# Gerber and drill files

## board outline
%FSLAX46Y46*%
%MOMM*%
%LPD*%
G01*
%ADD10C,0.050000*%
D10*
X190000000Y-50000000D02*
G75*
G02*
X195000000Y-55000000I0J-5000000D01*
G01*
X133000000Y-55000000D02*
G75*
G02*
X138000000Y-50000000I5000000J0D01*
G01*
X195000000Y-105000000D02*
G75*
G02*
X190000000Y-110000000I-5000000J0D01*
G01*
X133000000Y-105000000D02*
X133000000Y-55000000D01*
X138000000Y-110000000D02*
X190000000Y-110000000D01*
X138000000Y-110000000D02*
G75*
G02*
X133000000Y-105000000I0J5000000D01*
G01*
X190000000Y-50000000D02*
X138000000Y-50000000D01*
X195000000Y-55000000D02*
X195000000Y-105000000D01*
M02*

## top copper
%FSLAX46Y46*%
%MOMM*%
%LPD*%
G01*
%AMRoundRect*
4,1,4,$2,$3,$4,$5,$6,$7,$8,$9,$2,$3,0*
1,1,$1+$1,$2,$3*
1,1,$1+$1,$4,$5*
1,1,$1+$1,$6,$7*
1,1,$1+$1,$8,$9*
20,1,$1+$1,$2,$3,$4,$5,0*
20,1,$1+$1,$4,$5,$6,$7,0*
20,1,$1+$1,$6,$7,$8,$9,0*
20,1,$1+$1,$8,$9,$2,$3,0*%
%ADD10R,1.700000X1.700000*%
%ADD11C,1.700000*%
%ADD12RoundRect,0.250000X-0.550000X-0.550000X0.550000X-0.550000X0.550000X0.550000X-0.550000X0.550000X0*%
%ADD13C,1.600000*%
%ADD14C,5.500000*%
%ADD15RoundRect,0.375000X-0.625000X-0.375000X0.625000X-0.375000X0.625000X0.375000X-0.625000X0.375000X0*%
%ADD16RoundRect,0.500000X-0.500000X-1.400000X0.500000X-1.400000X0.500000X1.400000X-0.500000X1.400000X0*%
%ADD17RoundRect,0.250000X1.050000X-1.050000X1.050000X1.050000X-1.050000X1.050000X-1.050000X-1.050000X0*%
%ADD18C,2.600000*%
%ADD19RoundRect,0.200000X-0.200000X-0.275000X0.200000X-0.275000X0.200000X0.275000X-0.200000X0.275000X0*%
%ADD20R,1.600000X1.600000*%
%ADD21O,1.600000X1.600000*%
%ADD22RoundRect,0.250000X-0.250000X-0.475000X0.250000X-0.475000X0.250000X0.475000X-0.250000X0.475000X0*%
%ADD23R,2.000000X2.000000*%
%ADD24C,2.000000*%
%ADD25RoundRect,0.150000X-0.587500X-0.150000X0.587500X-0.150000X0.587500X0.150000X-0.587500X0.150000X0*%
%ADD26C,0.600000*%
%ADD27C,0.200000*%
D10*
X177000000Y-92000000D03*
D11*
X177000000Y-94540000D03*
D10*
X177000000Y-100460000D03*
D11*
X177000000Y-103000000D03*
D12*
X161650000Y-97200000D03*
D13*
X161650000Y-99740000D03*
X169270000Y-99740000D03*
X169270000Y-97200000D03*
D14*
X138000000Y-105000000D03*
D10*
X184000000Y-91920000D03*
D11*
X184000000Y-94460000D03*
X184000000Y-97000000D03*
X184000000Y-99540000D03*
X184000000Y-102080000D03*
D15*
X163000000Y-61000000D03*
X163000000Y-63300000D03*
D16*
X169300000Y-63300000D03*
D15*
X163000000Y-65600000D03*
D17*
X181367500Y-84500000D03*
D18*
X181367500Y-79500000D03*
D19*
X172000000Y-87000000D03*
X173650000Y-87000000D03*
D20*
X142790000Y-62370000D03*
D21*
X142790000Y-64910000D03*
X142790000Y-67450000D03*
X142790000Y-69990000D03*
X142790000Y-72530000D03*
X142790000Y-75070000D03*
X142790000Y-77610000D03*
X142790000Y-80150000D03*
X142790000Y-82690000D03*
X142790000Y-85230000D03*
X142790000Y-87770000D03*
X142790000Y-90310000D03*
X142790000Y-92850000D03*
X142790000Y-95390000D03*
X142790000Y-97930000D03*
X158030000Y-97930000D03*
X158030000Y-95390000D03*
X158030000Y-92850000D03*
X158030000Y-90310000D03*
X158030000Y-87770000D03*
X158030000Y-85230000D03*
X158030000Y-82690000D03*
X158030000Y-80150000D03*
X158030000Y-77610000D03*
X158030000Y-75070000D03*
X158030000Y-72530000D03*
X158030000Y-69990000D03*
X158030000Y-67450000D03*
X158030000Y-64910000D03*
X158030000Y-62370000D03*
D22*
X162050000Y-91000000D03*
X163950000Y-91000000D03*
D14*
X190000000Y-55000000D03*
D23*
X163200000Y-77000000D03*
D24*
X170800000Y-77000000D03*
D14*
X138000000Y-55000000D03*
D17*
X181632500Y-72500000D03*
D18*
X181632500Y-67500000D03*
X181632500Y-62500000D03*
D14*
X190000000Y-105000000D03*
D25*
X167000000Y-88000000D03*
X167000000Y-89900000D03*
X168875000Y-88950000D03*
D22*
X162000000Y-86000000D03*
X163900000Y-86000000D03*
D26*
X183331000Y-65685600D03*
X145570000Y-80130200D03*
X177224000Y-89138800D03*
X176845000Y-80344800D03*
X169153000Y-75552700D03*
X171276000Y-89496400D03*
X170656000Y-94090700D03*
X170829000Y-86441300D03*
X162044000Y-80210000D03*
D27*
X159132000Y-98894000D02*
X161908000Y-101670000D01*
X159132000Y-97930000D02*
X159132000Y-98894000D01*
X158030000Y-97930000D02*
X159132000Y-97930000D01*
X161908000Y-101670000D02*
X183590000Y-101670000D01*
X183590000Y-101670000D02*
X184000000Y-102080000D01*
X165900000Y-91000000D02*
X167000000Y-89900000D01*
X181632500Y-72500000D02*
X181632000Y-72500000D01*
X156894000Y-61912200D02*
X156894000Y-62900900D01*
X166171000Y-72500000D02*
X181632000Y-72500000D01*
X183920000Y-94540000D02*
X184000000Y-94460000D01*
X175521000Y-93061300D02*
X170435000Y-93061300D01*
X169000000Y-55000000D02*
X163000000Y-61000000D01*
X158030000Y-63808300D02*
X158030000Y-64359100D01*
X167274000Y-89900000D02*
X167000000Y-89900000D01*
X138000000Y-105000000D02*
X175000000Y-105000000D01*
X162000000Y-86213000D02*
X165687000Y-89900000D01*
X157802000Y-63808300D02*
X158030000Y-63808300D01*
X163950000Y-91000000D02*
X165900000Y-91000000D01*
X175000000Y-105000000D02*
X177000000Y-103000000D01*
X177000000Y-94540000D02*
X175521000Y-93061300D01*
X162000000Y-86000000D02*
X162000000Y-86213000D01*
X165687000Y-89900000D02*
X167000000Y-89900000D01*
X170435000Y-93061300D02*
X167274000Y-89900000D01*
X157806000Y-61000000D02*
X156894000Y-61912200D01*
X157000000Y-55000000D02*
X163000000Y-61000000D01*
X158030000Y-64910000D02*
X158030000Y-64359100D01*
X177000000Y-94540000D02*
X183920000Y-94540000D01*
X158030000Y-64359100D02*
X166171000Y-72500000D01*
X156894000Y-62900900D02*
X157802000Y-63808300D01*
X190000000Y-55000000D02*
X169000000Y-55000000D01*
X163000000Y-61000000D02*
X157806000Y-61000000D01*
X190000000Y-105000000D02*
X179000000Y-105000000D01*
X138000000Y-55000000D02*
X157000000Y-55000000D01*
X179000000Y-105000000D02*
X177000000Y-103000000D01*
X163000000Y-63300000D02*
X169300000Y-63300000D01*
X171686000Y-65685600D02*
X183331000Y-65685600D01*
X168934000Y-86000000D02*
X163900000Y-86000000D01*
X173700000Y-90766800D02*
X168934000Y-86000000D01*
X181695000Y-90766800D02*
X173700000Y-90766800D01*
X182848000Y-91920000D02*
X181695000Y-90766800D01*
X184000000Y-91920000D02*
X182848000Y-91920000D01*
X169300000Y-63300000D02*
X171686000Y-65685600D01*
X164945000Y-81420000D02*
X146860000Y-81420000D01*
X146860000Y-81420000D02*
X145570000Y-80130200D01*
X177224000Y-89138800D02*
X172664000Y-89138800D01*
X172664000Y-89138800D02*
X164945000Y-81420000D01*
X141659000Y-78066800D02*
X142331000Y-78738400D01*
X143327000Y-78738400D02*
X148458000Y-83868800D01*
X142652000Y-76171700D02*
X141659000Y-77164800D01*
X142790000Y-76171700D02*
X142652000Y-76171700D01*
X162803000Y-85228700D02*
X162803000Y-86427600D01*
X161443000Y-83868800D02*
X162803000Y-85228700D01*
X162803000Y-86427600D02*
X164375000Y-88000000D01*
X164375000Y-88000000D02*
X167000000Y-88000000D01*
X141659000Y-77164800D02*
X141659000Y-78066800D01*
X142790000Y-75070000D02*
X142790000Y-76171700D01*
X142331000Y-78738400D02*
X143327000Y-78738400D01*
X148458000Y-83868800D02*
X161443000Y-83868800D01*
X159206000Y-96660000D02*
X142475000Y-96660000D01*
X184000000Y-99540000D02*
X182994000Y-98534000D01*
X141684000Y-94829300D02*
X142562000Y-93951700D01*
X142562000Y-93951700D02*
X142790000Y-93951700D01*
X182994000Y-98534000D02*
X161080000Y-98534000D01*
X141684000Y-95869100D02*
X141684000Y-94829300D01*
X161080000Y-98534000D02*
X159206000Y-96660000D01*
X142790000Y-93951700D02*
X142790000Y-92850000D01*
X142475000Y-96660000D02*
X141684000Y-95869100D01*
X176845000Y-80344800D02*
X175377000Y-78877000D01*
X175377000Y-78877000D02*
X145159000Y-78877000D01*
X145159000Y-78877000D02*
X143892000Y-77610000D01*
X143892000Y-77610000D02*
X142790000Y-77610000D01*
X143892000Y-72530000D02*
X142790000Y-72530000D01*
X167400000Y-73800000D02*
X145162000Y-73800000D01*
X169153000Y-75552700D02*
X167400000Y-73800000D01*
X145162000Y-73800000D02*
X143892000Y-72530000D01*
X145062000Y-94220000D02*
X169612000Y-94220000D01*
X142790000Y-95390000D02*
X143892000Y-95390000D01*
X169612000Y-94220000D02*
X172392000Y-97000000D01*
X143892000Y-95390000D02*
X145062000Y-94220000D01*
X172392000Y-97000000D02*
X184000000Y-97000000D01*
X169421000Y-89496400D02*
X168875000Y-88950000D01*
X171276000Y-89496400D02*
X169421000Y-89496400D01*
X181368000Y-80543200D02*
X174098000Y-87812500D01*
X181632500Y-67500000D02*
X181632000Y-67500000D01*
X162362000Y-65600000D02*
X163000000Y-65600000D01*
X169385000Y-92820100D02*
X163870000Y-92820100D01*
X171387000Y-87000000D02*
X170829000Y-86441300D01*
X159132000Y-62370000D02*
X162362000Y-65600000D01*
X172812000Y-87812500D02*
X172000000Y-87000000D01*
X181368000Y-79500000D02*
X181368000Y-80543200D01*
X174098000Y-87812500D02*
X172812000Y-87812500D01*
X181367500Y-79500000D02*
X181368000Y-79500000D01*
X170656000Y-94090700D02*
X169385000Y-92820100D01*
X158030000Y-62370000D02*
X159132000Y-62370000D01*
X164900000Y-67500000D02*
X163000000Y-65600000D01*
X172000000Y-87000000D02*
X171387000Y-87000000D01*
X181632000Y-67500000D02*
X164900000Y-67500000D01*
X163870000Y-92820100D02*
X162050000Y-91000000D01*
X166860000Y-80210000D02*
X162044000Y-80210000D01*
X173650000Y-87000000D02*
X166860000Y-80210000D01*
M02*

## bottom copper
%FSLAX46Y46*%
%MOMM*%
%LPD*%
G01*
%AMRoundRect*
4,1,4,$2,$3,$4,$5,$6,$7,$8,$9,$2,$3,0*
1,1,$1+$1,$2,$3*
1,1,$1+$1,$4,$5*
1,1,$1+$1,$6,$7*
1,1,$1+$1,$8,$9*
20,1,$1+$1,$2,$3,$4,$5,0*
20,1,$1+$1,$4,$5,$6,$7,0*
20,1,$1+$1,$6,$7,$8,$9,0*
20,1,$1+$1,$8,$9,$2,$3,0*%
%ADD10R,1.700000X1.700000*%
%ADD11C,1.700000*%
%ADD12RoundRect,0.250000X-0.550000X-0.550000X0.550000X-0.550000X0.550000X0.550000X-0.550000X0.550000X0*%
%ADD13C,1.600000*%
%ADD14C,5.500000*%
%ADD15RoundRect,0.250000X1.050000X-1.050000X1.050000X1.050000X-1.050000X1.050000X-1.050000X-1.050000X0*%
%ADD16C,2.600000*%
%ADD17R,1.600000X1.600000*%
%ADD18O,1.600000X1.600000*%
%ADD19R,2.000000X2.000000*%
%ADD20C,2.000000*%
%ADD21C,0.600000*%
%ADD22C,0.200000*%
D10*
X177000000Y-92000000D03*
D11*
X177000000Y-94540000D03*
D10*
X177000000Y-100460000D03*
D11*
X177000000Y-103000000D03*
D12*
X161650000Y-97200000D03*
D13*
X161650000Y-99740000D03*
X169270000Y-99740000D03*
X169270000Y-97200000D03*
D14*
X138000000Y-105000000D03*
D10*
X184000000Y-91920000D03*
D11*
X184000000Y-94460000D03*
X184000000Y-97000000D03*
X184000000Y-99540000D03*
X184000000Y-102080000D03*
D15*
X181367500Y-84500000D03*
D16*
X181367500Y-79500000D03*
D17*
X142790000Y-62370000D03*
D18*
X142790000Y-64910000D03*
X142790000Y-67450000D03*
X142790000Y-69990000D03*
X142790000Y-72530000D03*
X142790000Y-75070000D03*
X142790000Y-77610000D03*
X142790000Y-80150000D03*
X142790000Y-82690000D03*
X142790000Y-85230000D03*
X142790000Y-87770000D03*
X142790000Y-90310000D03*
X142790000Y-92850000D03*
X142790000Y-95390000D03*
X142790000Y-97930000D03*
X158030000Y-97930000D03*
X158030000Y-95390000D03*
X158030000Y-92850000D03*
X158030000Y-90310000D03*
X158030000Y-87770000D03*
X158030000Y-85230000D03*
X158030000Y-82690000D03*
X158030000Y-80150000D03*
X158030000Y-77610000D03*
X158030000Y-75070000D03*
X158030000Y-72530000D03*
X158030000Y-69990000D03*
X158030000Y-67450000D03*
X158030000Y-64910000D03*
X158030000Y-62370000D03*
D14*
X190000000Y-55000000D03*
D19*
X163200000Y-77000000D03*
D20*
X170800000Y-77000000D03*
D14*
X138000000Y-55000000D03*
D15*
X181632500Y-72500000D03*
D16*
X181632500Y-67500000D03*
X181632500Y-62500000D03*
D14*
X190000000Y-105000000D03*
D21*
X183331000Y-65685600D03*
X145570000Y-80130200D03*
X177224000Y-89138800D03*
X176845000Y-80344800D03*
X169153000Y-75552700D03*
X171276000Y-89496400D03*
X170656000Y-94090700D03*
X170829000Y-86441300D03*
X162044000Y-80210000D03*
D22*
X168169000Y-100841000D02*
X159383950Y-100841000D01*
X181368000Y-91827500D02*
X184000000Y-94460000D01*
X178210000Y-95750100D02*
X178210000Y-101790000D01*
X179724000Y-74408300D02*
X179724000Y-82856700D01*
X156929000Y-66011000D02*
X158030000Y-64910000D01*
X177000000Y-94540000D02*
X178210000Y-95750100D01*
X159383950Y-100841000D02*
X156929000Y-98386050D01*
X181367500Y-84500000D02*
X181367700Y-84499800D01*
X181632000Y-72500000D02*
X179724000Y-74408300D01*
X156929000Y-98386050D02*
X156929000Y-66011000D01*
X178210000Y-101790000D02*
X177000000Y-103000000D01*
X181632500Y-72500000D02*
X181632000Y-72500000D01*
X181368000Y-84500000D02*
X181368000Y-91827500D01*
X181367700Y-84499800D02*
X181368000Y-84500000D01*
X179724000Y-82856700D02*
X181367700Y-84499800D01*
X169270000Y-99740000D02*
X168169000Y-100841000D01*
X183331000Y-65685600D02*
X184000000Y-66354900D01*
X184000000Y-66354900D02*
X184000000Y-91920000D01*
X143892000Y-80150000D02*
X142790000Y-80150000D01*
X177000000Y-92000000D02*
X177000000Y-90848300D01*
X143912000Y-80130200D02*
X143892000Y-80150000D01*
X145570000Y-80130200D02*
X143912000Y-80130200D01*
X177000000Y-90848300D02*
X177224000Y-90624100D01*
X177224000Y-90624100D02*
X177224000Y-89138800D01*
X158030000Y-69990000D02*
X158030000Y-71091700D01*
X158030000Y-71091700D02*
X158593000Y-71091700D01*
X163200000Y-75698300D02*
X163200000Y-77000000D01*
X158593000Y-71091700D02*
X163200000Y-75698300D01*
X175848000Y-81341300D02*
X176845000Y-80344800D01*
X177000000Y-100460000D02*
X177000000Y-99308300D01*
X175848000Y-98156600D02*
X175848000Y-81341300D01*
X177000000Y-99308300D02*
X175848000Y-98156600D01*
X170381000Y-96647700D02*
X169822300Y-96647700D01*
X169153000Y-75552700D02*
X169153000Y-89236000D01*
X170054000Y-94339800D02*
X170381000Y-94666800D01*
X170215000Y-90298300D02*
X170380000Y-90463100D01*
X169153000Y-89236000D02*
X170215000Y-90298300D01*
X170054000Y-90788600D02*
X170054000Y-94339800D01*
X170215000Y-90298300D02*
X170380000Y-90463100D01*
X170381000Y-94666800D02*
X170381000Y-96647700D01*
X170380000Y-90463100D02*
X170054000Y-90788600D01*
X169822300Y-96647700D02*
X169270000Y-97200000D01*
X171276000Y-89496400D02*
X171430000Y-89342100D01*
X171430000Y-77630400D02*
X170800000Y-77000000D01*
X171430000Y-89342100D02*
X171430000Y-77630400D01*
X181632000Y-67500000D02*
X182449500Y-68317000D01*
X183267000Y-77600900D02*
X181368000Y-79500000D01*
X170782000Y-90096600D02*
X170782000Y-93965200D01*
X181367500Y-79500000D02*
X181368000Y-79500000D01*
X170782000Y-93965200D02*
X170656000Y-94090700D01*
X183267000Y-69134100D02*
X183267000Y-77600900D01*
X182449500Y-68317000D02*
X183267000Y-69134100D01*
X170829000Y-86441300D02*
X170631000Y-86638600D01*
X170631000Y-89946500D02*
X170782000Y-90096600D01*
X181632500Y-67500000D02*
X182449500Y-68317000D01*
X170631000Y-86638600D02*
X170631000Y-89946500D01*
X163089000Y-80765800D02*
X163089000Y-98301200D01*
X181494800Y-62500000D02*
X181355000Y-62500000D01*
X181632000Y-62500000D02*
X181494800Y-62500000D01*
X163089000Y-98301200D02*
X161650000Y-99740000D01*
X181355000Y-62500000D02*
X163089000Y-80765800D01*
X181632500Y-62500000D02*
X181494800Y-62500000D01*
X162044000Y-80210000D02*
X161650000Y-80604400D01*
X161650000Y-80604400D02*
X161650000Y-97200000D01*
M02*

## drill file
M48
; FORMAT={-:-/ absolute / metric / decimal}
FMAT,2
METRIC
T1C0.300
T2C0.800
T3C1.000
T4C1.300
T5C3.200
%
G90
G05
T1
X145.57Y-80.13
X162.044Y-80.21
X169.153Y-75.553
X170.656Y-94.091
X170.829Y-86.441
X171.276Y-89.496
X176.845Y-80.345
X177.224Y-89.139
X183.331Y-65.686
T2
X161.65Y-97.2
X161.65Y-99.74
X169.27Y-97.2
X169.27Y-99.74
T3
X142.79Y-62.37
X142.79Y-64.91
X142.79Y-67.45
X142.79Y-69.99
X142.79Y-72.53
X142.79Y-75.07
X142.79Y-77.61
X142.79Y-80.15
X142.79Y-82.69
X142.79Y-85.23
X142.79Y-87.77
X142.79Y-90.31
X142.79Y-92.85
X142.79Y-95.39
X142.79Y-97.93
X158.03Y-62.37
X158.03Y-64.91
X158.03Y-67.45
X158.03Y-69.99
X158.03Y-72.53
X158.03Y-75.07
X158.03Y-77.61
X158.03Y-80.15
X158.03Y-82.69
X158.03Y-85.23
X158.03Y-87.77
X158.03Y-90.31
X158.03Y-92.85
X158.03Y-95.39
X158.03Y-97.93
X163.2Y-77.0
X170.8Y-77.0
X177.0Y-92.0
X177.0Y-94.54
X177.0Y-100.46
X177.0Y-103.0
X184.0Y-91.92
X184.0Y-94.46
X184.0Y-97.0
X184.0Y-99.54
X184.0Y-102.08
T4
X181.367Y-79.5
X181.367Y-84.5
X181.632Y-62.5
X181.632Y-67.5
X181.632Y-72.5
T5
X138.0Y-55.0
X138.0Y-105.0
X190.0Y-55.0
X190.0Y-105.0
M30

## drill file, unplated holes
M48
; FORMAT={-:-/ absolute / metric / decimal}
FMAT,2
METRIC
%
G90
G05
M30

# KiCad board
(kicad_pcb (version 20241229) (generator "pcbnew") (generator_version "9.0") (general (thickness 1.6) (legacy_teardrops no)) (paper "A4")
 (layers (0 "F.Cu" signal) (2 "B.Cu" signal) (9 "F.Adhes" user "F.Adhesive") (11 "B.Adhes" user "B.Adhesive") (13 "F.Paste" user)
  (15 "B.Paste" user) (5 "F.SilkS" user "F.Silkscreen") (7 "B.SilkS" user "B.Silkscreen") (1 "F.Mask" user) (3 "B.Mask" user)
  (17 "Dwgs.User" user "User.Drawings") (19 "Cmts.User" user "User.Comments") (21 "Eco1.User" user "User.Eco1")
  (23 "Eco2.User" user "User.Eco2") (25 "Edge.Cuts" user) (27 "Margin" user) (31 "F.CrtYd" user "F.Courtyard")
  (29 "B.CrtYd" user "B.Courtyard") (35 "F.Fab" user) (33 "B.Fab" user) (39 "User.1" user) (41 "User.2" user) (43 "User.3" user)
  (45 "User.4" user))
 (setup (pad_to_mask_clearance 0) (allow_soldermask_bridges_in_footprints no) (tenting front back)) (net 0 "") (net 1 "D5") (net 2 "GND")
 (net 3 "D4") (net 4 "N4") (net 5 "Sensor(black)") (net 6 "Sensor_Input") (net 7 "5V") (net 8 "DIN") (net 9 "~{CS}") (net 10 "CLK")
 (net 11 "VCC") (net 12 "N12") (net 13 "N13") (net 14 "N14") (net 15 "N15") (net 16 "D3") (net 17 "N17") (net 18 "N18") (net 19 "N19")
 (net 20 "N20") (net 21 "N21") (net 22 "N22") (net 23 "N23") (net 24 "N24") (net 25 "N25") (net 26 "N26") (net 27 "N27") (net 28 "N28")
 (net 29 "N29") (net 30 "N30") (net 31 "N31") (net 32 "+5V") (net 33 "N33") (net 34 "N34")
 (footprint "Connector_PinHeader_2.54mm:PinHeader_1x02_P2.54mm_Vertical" (layer "F.Cu") (at 177 92)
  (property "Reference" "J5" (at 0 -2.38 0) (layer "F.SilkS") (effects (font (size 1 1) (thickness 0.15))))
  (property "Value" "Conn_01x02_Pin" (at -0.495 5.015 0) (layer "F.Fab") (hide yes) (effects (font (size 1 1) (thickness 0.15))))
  (pad "1" thru_hole rect (at 0 0) (size 1.7 1.7) (drill 1) (layers "*.Cu" "*.Mask") (remove_unused_layers no) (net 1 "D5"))
  (pad "2" thru_hole circle (at 0 2.54) (size 1.7 1.7) (drill 1) (layers "*.Cu" "*.Mask") (remove_unused_layers no) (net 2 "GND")))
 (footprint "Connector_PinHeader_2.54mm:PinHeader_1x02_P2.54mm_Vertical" (layer "F.Cu") (at 177 100.46)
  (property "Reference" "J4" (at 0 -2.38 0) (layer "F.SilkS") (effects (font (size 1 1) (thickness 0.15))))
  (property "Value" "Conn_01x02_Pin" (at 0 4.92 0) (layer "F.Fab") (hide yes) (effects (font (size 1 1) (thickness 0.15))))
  (pad "1" thru_hole rect (at 0 0) (size 1.7 1.7) (drill 1) (layers "*.Cu" "*.Mask") (remove_unused_layers no) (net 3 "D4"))
  (pad "2" thru_hole circle (at 0 2.54) (size 1.7 1.7) (drill 1) (layers "*.Cu" "*.Mask") (remove_unused_layers no) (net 2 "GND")))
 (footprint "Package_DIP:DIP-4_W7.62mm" (layer "F.Cu") (at 161.65 97.2)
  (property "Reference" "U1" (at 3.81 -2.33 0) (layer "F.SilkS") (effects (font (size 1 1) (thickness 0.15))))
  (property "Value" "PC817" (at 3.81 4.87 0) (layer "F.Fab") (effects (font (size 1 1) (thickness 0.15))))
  (pad "1" thru_hole roundrect (at 0 0) (size 1.6 1.6) (drill 0.8) (layers "*.Cu" "*.Mask") (remove_unused_layers no)
   (roundrect_rratio 0.15625) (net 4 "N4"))
  (pad "2" thru_hole circle (at 0 2.54) (size 1.6 1.6) (drill 0.8) (layers "*.Cu" "*.Mask") (remove_unused_layers no)
   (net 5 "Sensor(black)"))
  (pad "3" thru_hole circle (at 7.62 2.54) (size 1.6 1.6) (drill 0.8) (layers "*.Cu" "*.Mask") (remove_unused_layers no) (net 2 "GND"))
  (pad "4" thru_hole circle (at 7.62 0) (size 1.6 1.6) (drill 0.8) (layers "*.Cu" "*.Mask") (remove_unused_layers no) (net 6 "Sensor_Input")))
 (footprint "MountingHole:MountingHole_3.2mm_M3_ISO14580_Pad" (layer "F.Cu") (at 138 105)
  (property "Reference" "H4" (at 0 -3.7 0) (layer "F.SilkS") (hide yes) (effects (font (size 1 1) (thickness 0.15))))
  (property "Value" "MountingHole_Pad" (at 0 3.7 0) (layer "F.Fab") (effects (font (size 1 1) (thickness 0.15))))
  (pad "1" thru_hole circle (at 0 0) (size 5.5 5.5) (drill 3.2) (layers "*.Cu" "*.Mask") (remove_unused_layers no) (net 2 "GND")
   (zone_connect 2)))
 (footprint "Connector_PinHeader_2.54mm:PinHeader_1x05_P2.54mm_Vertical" (layer "F.Cu") (at 184 91.92)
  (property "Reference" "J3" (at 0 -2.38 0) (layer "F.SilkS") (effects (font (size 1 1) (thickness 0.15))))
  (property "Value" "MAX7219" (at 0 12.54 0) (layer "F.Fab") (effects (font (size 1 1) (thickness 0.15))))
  (pad "1" thru_hole rect (at 0 0) (size 1.7 1.7) (drill 1) (layers "*.Cu" "*.Mask") (remove_unused_layers no) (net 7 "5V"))
  (pad "2" thru_hole circle (at 0 2.54) (size 1.7 1.7) (drill 1) (layers "*.Cu" "*.Mask") (remove_unused_layers no) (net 2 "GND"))
  (pad "3" thru_hole circle (at 0 5.08) (size 1.7 1.7) (drill 1) (layers "*.Cu" "*.Mask") (remove_unused_layers no) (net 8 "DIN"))
  (pad "4" thru_hole circle (at 0 7.62) (size 1.7 1.7) (drill 1) (layers "*.Cu" "*.Mask") (remove_unused_layers no) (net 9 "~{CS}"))
  (pad "5" thru_hole circle (at 0 10.16) (size 1.7 1.7) (drill 1) (layers "*.Cu" "*.Mask") (remove_unused_layers no) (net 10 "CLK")))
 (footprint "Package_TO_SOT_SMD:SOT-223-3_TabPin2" (layer "F.Cu") (at 166.15 63.3)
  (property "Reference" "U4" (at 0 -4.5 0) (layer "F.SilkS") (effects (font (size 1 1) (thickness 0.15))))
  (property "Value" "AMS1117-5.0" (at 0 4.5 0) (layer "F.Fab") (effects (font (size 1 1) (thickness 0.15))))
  (pad "1" smd roundrect (at -3.15 -2.3) (size 2 1.5) (layers "F.Cu" "F.Mask" "F.Paste") (roundrect_rratio 0.25) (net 2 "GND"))
  (pad "2" smd roundrect (at -3.15 0) (size 2 1.5) (layers "F.Cu" "F.Mask" "F.Paste") (roundrect_rratio 0.25) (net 7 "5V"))
  (pad "2" smd roundrect (at 3.15 0) (size 2 3.8) (layers "F.Cu" "F.Mask" "F.Paste") (roundrect_rratio 0.25) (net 7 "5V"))
  (pad "3" smd roundrect (at -3.15 2.3) (size 2 1.5) (layers "F.Cu" "F.Mask" "F.Paste") (roundrect_rratio 0.25) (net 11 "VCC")))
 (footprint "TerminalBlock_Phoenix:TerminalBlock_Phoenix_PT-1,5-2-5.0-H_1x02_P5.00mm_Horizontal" (layer "F.Cu") (at 181.3675 84.5 90)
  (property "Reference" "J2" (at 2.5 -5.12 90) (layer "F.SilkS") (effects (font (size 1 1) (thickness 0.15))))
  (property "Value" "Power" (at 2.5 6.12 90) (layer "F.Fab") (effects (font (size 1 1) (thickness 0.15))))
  (pad "1" thru_hole roundrect (at 0 0 90) (size 2.6 2.6) (drill 1.3) (layers "*.Cu" "*.Mask") (remove_unused_layers no)
   (roundrect_rratio 0.096154) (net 2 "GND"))
  (pad "2" thru_hole circle (at 5 0 90) (size 2.6 2.6) (drill 1.3) (layers "*.Cu" "*.Mask") (remove_unused_layers no) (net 11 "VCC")))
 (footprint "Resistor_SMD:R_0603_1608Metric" (layer "F.Cu") (at 172.825 87)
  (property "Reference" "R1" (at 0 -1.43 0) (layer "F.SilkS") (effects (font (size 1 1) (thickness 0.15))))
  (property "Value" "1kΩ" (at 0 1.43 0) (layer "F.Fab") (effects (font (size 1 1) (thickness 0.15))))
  (pad "1" smd roundrect (at -0.825 0) (size 0.8 0.95) (layers "F.Cu" "F.Mask" "F.Paste") (roundrect_rratio 0.25) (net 11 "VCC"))
  (pad "2" smd roundrect (at 0.825 0) (size 0.8 0.95) (layers "F.Cu" "F.Mask" "F.Paste") (roundrect_rratio 0.25) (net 4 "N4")))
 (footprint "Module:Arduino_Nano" (layer "F.Cu") (at 142.79 62.37)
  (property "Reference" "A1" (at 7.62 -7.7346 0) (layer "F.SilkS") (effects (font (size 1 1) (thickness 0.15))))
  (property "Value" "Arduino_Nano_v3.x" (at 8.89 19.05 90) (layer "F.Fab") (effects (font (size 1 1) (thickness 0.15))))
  (pad "1" thru_hole rect (at 0 0) (size 1.6 1.6) (drill 1) (layers "*.Cu" "*.Mask") (remove_unused_layers no) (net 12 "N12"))
  (pad "2" thru_hole oval (at 0 2.54) (size 1.6 1.6) (drill 1) (layers "*.Cu" "*.Mask") (remove_unused_layers no) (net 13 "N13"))
  (pad "3" thru_hole oval (at 0 5.08) (size 1.6 1.6) (drill 1) (layers "*.Cu" "*.Mask") (remove_unused_layers no) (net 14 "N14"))
  (pad "4" thru_hole oval (at 0 7.62) (size 1.6 1.6) (drill 1) (layers "*.Cu" "*.Mask") (remove_unused_layers no) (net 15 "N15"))
  (pad "5" thru_hole oval (at 0 10.16) (size 1.6 1.6) (drill 1) (layers "*.Cu" "*.Mask") (remove_unused_layers no) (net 6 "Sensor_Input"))
  (pad "6" thru_hole oval (at 0 12.7) (size 1.6 1.6) (drill 1) (layers "*.Cu" "*.Mask") (remove_unused_layers no) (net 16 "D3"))
  (pad "7" thru_hole oval (at 0 15.24) (size 1.6 1.6) (drill 1) (layers "*.Cu" "*.Mask") (remove_unused_layers no) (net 3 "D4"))
  (pad "8" thru_hole oval (at 0 17.78) (size 1.6 1.6) (drill 1) (layers "*.Cu" "*.Mask") (remove_unused_layers no) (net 1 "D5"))
  (pad "9" thru_hole oval (at 0 20.32) (size 1.6 1.6) (drill 1) (layers "*.Cu" "*.Mask") (remove_unused_layers no) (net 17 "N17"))
  (pad "10" thru_hole oval (at 0 22.86) (size 1.6 1.6) (drill 1) (layers "*.Cu" "*.Mask") (remove_unused_layers no) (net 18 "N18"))
  (pad "11" thru_hole oval (at 0 25.4) (size 1.6 1.6) (drill 1) (layers "*.Cu" "*.Mask") (remove_unused_layers no) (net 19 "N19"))
  (pad "12" thru_hole oval (at 0 27.94) (size 1.6 1.6) (drill 1) (layers "*.Cu" "*.Mask") (remove_unused_layers no) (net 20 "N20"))
  (pad "13" thru_hole oval (at 0 30.48) (size 1.6 1.6) (drill 1) (layers "*.Cu" "*.Mask") (remove_unused_layers no) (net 9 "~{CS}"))
  (pad "14" thru_hole oval (at 0 33.02) (size 1.6 1.6) (drill 1) (layers "*.Cu" "*.Mask") (remove_unused_layers no) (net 8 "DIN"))
  (pad "15" thru_hole oval (at 0 35.56) (size 1.6 1.6) (drill 1) (layers "*.Cu" "*.Mask") (remove_unused_layers no) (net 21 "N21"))
  (pad "16" thru_hole oval (at 15.24 35.56) (size 1.6 1.6) (drill 1) (layers "*.Cu" "*.Mask") (remove_unused_layers no) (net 10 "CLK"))
  (pad "17" thru_hole oval (at 15.24 33.02) (size 1.6 1.6) (drill 1) (layers "*.Cu" "*.Mask") (remove_unused_layers no) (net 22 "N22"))
  (pad "18" thru_hole oval (at 15.24 30.48) (size 1.6 1.6) (drill 1) (layers "*.Cu" "*.Mask") (remove_unused_layers no) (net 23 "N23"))
  (pad "19" thru_hole oval (at 15.24 27.94) (size 1.6 1.6) (drill 1) (layers "*.Cu" "*.Mask") (remove_unused_layers no) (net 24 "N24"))
  (pad "20" thru_hole oval (at 15.24 25.4) (size 1.6 1.6) (drill 1) (layers "*.Cu" "*.Mask") (remove_unused_layers no) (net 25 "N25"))
  (pad "21" thru_hole oval (at 15.24 22.86) (size 1.6 1.6) (drill 1) (layers "*.Cu" "*.Mask") (remove_unused_layers no) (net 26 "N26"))
  (pad "22" thru_hole oval (at 15.24 20.32) (size 1.6 1.6) (drill 1) (layers "*.Cu" "*.Mask") (remove_unused_layers no) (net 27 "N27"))
  (pad "23" thru_hole oval (at 15.24 17.78) (size 1.6 1.6) (drill 1) (layers "*.Cu" "*.Mask") (remove_unused_layers no) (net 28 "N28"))
  (pad "24" thru_hole oval (at 15.24 15.24) (size 1.6 1.6) (drill 1) (layers "*.Cu" "*.Mask") (remove_unused_layers no) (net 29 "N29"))
  (pad "25" thru_hole oval (at 15.24 12.7) (size 1.6 1.6) (drill 1) (layers "*.Cu" "*.Mask") (remove_unused_layers no) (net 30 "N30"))
  (pad "26" thru_hole oval (at 15.24 10.16) (size 1.6 1.6) (drill 1) (layers "*.Cu" "*.Mask") (remove_unused_layers no) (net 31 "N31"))
  (pad "27" thru_hole oval (at 15.24 7.62) (size 1.6 1.6) (drill 1) (layers "*.Cu" "*.Mask") (remove_unused_layers no) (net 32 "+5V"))
  (pad "28" thru_hole oval (at 15.24 5.08) (size 1.6 1.6) (drill 1) (layers "*.Cu" "*.Mask") (remove_unused_layers no) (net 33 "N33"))
  (pad "29" thru_hole oval (at 15.24 2.54) (size 1.6 1.6) (drill 1) (layers "*.Cu" "*.Mask") (remove_unused_layers no) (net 2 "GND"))
  (pad "30" thru_hole oval (at 15.24 0) (size 1.6 1.6) (drill 1) (layers "*.Cu" "*.Mask") (remove_unused_layers no) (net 11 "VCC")))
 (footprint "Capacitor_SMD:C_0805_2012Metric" (layer "F.Cu") (at 163 91)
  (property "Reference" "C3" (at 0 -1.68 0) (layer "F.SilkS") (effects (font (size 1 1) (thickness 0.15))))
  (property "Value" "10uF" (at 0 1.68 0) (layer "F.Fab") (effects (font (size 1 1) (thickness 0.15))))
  (pad "1" smd roundrect (at -0.95 0) (size 1 1.45) (layers "F.Cu" "F.Mask" "F.Paste") (roundrect_rratio 0.25) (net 11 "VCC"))
  (pad "2" smd roundrect (at 0.95 0) (size 1 1.45) (layers "F.Cu" "F.Mask" "F.Paste") (roundrect_rratio 0.25) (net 2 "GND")))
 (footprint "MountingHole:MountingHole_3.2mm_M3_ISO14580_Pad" (layer "F.Cu") (at 190 55)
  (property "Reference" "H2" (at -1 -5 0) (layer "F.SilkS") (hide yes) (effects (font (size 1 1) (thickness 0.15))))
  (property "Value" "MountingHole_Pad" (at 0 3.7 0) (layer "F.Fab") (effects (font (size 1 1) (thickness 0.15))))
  (pad "1" thru_hole circle (at 0 0) (size 5.5 5.5) (drill 3.2) (layers "*.Cu" "*.Mask") (remove_unused_layers no) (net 2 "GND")
   (zone_connect 2)))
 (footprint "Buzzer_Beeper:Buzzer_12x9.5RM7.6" (layer "F.Cu") (at 163.2 77)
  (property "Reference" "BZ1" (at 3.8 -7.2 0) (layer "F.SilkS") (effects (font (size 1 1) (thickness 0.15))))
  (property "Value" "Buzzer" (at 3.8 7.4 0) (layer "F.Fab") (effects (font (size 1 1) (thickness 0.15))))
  (pad "1" thru_hole rect (at 0 0) (size 2 2) (drill 1) (layers "*.Cu" "*.Mask") (remove_unused_layers no) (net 32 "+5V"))
  (pad "2" thru_hole circle (at 7.6 0) (size 2 2) (drill 1) (layers "*.Cu" "*.Mask") (remove_unused_layers no) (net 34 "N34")))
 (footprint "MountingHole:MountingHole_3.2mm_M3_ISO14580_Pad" (layer "F.Cu") (at 138 55)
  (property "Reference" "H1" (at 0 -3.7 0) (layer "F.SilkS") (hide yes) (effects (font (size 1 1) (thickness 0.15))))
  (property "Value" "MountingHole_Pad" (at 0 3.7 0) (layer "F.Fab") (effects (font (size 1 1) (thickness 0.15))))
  (pad "1" thru_hole circle (at 0 0) (size 5.5 5.5) (drill 3.2) (layers "*.Cu" "*.Mask") (remove_unused_layers no) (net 2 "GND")
   (zone_connect 2)))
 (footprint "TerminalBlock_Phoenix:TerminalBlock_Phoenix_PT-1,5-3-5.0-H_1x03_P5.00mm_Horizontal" (layer "F.Cu") (at 181.6325 72.5 90)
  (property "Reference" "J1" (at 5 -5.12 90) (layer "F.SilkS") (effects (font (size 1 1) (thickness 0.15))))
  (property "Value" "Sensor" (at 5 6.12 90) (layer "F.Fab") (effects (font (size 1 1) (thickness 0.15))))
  (pad "1" thru_hole roundrect (at 0 0 90) (size 2.6 2.6) (drill 1.3) (layers "*.Cu" "*.Mask") (remove_unused_layers no)
   (roundrect_rratio 0.096154) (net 2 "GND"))
  (pad "2" thru_hole circle (at 5 0 90) (size 2.6 2.6) (drill 1.3) (layers "*.Cu" "*.Mask") (remove_unused_layers no) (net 11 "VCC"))
  (pad "3" thru_hole circle (at 10 0 90) (size 2.6 2.6) (drill 1.3) (layers "*.Cu" "*.Mask") (remove_unused_layers no)
   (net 5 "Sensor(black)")))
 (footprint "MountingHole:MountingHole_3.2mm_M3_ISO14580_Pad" (layer "F.Cu") (at 190 105)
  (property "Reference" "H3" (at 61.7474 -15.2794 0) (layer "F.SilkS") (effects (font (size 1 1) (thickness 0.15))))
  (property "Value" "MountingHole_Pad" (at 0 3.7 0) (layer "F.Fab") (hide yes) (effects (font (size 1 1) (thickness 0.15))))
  (pad "1" thru_hole circle (at 0 0) (size 5.5 5.5) (drill 3.2) (layers "*.Cu" "*.Mask") (remove_unused_layers no) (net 2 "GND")
   (zone_connect 2)))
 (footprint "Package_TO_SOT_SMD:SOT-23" (layer "F.Cu") (at 167.9375 88.95)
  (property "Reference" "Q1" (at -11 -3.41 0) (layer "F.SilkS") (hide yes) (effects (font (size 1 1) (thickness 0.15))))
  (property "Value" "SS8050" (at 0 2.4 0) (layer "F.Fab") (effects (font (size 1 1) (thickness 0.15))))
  (pad "1" smd roundrect (at -0.9375 -0.95) (size 1.475 0.6) (layers "F.Cu" "F.Mask" "F.Paste") (roundrect_rratio 0.25) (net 16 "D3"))
  (pad "2" smd roundrect (at -0.9375 0.95) (size 1.475 0.6) (layers "F.Cu" "F.Mask" "F.Paste") (roundrect_rratio 0.25) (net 2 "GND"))
  (pad "3" smd roundrect (at 0.9375 0) (size 1.475 0.6) (layers "F.Cu" "F.Mask" "F.Paste") (roundrect_rratio 0.25) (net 34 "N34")))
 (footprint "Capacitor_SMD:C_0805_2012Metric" (layer "F.Cu") (at 162.95 86)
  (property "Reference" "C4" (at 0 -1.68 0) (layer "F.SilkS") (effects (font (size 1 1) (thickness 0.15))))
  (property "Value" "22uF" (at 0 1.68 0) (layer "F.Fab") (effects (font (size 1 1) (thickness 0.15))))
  (pad "1" smd roundrect (at -0.95 0) (size 1 1.45) (layers "F.Cu" "F.Mask" "F.Paste") (roundrect_rratio 0.25) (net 2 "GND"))
  (pad "2" smd roundrect (at 0.95 0) (size 1 1.45) (layers "F.Cu" "F.Mask" "F.Paste") (roundrect_rratio 0.25) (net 7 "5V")))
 (gr_arc (start 190 50) (mid 193.535534 51.464466) (end 195 55) (stroke (width 0.05) (type default)) (layer "Edge.Cuts"))
 (gr_arc (start 133 55) (mid 134.464466 51.464466) (end 138 50) (stroke (width 0.05) (type default)) (layer "Edge.Cuts"))
 (gr_arc (start 195 105) (mid 193.535534 108.535534) (end 190 110) (stroke (width 0.05) (type default)) (layer "Edge.Cuts"))
 (gr_line (start 133 105) (end 133 55) (stroke (width 0.05) (type default)) (layer "Edge.Cuts"))
 (gr_line (start 138 110) (end 190 110) (stroke (width 0.05) (type default)) (layer "Edge.Cuts"))
 (gr_arc (start 138 110) (mid 134.464466 108.535534) (end 133 105) (stroke (width 0.05) (type default)) (layer "Edge.Cuts"))
 (gr_line (start 190 50) (end 138 50) (stroke (width 0.05) (type default)) (layer "Edge.Cuts"))
 (gr_line (start 195 55) (end 195 105) (stroke (width 0.05) (type default)) (layer "Edge.Cuts"))
 (segment (start 159.132 98.894) (end 161.908 101.67) (width 0.2) (layer "F.Cu") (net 10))
 (segment (start 159.132 97.93) (end 159.132 98.894) (width 0.2) (layer "F.Cu") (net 10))
 (segment (start 158.03 97.93) (end 159.132 97.93) (width 0.2) (layer "F.Cu") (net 10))
 (segment (start 161.908 101.67) (end 183.59 101.67) (width 0.2) (layer "F.Cu") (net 10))
 (segment (start 183.59 101.67) (end 184 102.08) (width 0.2) (layer "F.Cu") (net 10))
 (segment (start 165.9 91) (end 167 89.9) (width 0.2) (layer "F.Cu") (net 2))
 (segment (start 181.6325 72.5) (end 181.632 72.5) (width 0.2) (layer "F.Cu") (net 2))
 (segment (start 156.894 61.9122) (end 156.894 62.9009) (width 0.2) (layer "F.Cu") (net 2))
 (segment (start 166.171 72.5) (end 181.632 72.5) (width 0.2) (layer "F.Cu") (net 2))
 (segment (start 183.92 94.54) (end 184 94.46) (width 0.2) (layer "F.Cu") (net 2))
 (segment (start 175.521 93.0613) (end 170.435 93.0613) (width 0.2) (layer "F.Cu") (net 2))
 (segment (start 169 55) (end 163 61) (width 0.2) (layer "F.Cu") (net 2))
 (segment (start 158.03 63.8083) (end 158.03 64.3591) (width 0.2) (layer "F.Cu") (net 2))
 (segment (start 167.274 89.9) (end 167 89.9) (width 0.2) (layer "F.Cu") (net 2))
 (segment (start 138 105) (end 175 105) (width 0.2) (layer "F.Cu") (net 2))
 (segment (start 162 86.213) (end 165.687 89.9) (width 0.2) (layer "F.Cu") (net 2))
 (segment (start 157.802 63.8083) (end 158.03 63.8083) (width 0.2) (layer "F.Cu") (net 2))
 (segment (start 163.95 91) (end 165.9 91) (width 0.2) (layer "F.Cu") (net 2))
 (segment (start 175 105) (end 177 103) (width 0.2) (layer "F.Cu") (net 2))
 (segment (start 177 94.54) (end 175.521 93.0613) (width 0.2) (layer "F.Cu") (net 2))
 (segment (start 162 86) (end 162 86.213) (width 0.2) (layer "F.Cu") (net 2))
 (segment (start 165.687 89.9) (end 167 89.9) (width 0.2) (layer "F.Cu") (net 2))
 (segment (start 170.435 93.0613) (end 167.274 89.9) (width 0.2) (layer "F.Cu") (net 2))
 (segment (start 157.806 61) (end 156.894 61.9122) (width 0.2) (layer "F.Cu") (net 2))
 (segment (start 157 55) (end 163 61) (width 0.2) (layer "F.Cu") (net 2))
 (segment (start 158.03 64.91) (end 158.03 64.3591) (width 0.2) (layer "F.Cu") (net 2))
 (segment (start 177 94.54) (end 183.92 94.54) (width 0.2) (layer "F.Cu") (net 2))
 (segment (start 158.03 64.3591) (end 166.171 72.5) (width 0.2) (layer "F.Cu") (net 2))
 (segment (start 156.894 62.9009) (end 157.802 63.8083) (width 0.2) (layer "F.Cu") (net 2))
 (segment (start 190 55) (end 169 55) (width 0.2) (layer "F.Cu") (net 2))
 (segment (start 163 61) (end 157.806 61) (width 0.2) (layer "F.Cu") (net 2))
 (segment (start 190 105) (end 179 105) (width 0.2) (layer "F.Cu") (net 2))
 (segment (start 138 55) (end 157 55) (width 0.2) (layer "F.Cu") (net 2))
 (segment (start 179 105) (end 177 103) (width 0.2) (layer "F.Cu") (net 2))
 (segment (start 168.169 100.841) (end 159.38395 100.841) (width 0.2) (layer "B.Cu") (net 2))
 (segment (start 181.368 91.8275) (end 184 94.46) (width 0.2) (layer "B.Cu") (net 2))
 (segment (start 178.21 95.7501) (end 178.21 101.79) (width 0.2) (layer "B.Cu") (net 2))
 (segment (start 179.724 74.4083) (end 179.724 82.8567) (width 0.2) (layer "B.Cu") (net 2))
 (segment (start 156.929 66.011) (end 158.03 64.91) (width 0.2) (layer "B.Cu") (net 2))
 (segment (start 177 94.54) (end 178.21 95.7501) (width 0.2) (layer "B.Cu") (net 2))
 (segment (start 159.38395 100.841) (end 156.929 98.38605) (width 0.2) (layer "B.Cu") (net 2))
 (segment (start 181.3675 84.5) (end 181.3677 84.4998) (width 0.2) (layer "B.Cu") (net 2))
 (segment (start 181.632 72.5) (end 179.724 74.4083) (width 0.2) (layer "B.Cu") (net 2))
 (segment (start 156.929 98.38605) (end 156.929 66.011) (width 0.2) (layer "B.Cu") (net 2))
 (segment (start 178.21 101.79) (end 177 103) (width 0.2) (layer "B.Cu") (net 2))
 (segment (start 181.6325 72.5) (end 181.632 72.5) (width 0.2) (layer "B.Cu") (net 2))
 (segment (start 181.368 84.5) (end 181.368 91.8275) (width 0.2) (layer "B.Cu") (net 2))
 (segment (start 181.3677 84.4998) (end 181.368 84.5) (width 0.2) (layer "B.Cu") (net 2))
 (segment (start 179.724 82.8567) (end 181.3677 84.4998) (width 0.2) (layer "B.Cu") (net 2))
 (segment (start 169.27 99.74) (end 168.169 100.841) (width 0.2) (layer "B.Cu") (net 2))
 (segment (start 163 63.3) (end 169.3 63.3) (width 0.2) (layer "F.Cu") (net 7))
 (segment (start 171.686 65.6856) (end 183.331 65.6856) (width 0.2) (layer "F.Cu") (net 7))
 (segment (start 168.934 86) (end 163.9 86) (width 0.2) (layer "F.Cu") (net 7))
 (segment (start 173.7 90.7668) (end 168.934 86) (width 0.2) (layer "F.Cu") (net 7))
 (segment (start 181.695 90.7668) (end 173.7 90.7668) (width 0.2) (layer "F.Cu") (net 7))
 (segment (start 182.848 91.92) (end 181.695 90.7668) (width 0.2) (layer "F.Cu") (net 7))
 (segment (start 184 91.92) (end 182.848 91.92) (width 0.2) (layer "F.Cu") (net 7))
 (segment (start 169.3 63.3) (end 171.686 65.6856) (width 0.2) (layer "F.Cu") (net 7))
 (via (at 183.331 65.6856) (size 0.6) (drill 0.3) (layers "F.Cu" "B.Cu") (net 7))
 (segment (start 183.331 65.6856) (end 184 66.3549) (width 0.2) (layer "B.Cu") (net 7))
 (segment (start 184 66.3549) (end 184 91.92) (width 0.2) (layer "B.Cu") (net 7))
 (segment (start 164.945 81.42) (end 146.86 81.42) (width 0.2) (layer "F.Cu") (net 1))
 (segment (start 146.86 81.42) (end 145.57 80.1302) (width 0.2) (layer "F.Cu") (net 1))
 (segment (start 177.224 89.1388) (end 172.664 89.1388) (width 0.2) (layer "F.Cu") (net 1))
 (segment (start 172.664 89.1388) (end 164.945 81.42) (width 0.2) (layer "F.Cu") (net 1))
 (via (at 145.57 80.1302) (size 0.6) (drill 0.3) (layers "F.Cu" "B.Cu") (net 1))
 (via (at 177.224 89.1388) (size 0.6) (drill 0.3) (layers "F.Cu" "B.Cu") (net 1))
 (segment (start 143.892 80.15) (end 142.79 80.15) (width 0.2) (layer "B.Cu") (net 1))
 (segment (start 177 92) (end 177 90.8483) (width 0.2) (layer "B.Cu") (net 1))
 (segment (start 143.912 80.1302) (end 143.892 80.15) (width 0.2) (layer "B.Cu") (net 1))
 (segment (start 145.57 80.1302) (end 143.912 80.1302) (width 0.2) (layer "B.Cu") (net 1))
 (segment (start 177 90.8483) (end 177.224 90.6241) (width 0.2) (layer "B.Cu") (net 1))
 (segment (start 177.224 90.6241) (end 177.224 89.1388) (width 0.2) (layer "B.Cu") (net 1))
 (segment (start 141.659 78.0668) (end 142.331 78.7384) (width 0.2) (layer "F.Cu") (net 16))
 (segment (start 143.327 78.7384) (end 148.458 83.8688) (width 0.2) (layer "F.Cu") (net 16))
 (segment (start 142.652 76.1717) (end 141.659 77.1648) (width 0.2) (layer "F.Cu") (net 16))
 (segment (start 142.79 76.1717) (end 142.652 76.1717) (width 0.2) (layer "F.Cu") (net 16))
 (segment (start 162.803 85.2287) (end 162.803 86.4276) (width 0.2) (layer "F.Cu") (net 16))
 (segment (start 161.443 83.8688) (end 162.803 85.2287) (width 0.2) (layer "F.Cu") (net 16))
 (segment (start 162.803 86.4276) (end 164.375 88) (width 0.2) (layer "F.Cu") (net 16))
 (segment (start 164.375 88) (end 167 88) (width 0.2) (layer "F.Cu") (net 16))
 (segment (start 141.659 77.1648) (end 141.659 78.0668) (width 0.2) (layer "F.Cu") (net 16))
 (segment (start 142.79 75.07) (end 142.79 76.1717) (width 0.2) (layer "F.Cu") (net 16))
 (segment (start 142.331 78.7384) (end 143.327 78.7384) (width 0.2) (layer "F.Cu") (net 16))
 (segment (start 148.458 83.8688) (end 161.443 83.8688) (width 0.2) (layer "F.Cu") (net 16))
 (segment (start 158.03 69.99) (end 158.03 71.0917) (width 0.2) (layer "B.Cu") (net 32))
 (segment (start 158.03 71.0917) (end 158.593 71.0917) (width 0.2) (layer "B.Cu") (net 32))
 (segment (start 163.2 75.6983) (end 163.2 77) (width 0.2) (layer "B.Cu") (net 32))
 (segment (start 158.593 71.0917) (end 163.2 75.6983) (width 0.2) (layer "B.Cu") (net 32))
 (segment (start 159.206 96.66) (end 142.475 96.66) (width 0.2) (layer "F.Cu") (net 9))
 (segment (start 184 99.54) (end 182.994 98.534) (width 0.2) (layer "F.Cu") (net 9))
 (segment (start 141.684 94.8293) (end 142.562 93.9517) (width 0.2) (layer "F.Cu") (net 9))
 (segment (start 142.562 93.9517) (end 142.79 93.9517) (width 0.2) (layer "F.Cu") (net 9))
 (segment (start 182.994 98.534) (end 161.08 98.534) (width 0.2) (layer "F.Cu") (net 9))
 (segment (start 141.684 95.8691) (end 141.684 94.8293) (width 0.2) (layer "F.Cu") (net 9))
 (segment (start 161.08 98.534) (end 159.206 96.66) (width 0.2) (layer "F.Cu") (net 9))
 (segment (start 142.79 93.9517) (end 142.79 92.85) (width 0.2) (layer "F.Cu") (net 9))
 (segment (start 142.475 96.66) (end 141.684 95.8691) (width 0.2) (layer "F.Cu") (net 9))
 (segment (start 176.845 80.3448) (end 175.377 78.877) (width 0.2) (layer "F.Cu") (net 3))
 (segment (start 175.377 78.877) (end 145.159 78.877) (width 0.2) (layer "F.Cu") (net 3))
 (segment (start 145.159 78.877) (end 143.892 77.61) (width 0.2) (layer "F.Cu") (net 3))
 (segment (start 143.892 77.61) (end 142.79 77.61) (width 0.2) (layer "F.Cu") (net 3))
 (via (at 176.845 80.3448) (size 0.6) (drill 0.3) (layers "F.Cu" "B.Cu") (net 3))
 (segment (start 175.848 81.3413) (end 176.845 80.3448) (width 0.2) (layer "B.Cu") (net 3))
 (segment (start 177 100.46) (end 177 99.3083) (width 0.2) (layer "B.Cu") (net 3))
 (segment (start 175.848 98.1566) (end 175.848 81.3413) (width 0.2) (layer "B.Cu") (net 3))
 (segment (start 177 99.3083) (end 175.848 98.1566) (width 0.2) (layer "B.Cu") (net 3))
 (segment (start 143.892 72.53) (end 142.79 72.53) (width 0.2) (layer "F.Cu") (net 6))
 (segment (start 167.4 73.8) (end 145.162 73.8) (width 0.2) (layer "F.Cu") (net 6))
 (segment (start 169.153 75.5527) (end 167.4 73.8) (width 0.2) (layer "F.Cu") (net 6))
 (segment (start 145.162 73.8) (end 143.892 72.53) (width 0.2) (layer "F.Cu") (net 6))
 (via (at 169.153 75.5527) (size 0.6) (drill 0.3) (layers "F.Cu" "B.Cu") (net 6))
 (segment (start 170.381 96.6477) (end 169.8223 96.6477) (width 0.2) (layer "B.Cu") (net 6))
 (segment (start 169.153 75.5527) (end 169.153 89.236) (width 0.2) (layer "B.Cu") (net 6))
 (segment (start 170.054 94.3398) (end 170.381 94.6668) (width 0.2) (layer "B.Cu") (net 6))
 (segment (start 170.215 90.2983) (end 170.38 90.4631) (width 0.2) (layer "B.Cu") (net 6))
 (segment (start 169.153 89.236) (end 170.215 90.2983) (width 0.2) (layer "B.Cu") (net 6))
 (segment (start 170.054 90.7886) (end 170.054 94.3398) (width 0.2) (layer "B.Cu") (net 6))
 (segment (start 170.215 90.2983) (end 170.38 90.4631) (width 0.2) (layer "B.Cu") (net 6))
 (segment (start 170.381 94.6668) (end 170.381 96.6477) (width 0.2) (layer "B.Cu") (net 6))
 (segment (start 170.38 90.4631) (end 170.054 90.7886) (width 0.2) (layer "B.Cu") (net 6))
 (segment (start 169.8223 96.6477) (end 169.27 97.2) (width 0.2) (layer "B.Cu") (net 6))
 (segment (start 145.062 94.22) (end 169.612 94.22) (width 0.2) (layer "F.Cu") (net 8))
 (segment (start 142.79 95.39) (end 143.892 95.39) (width 0.2) (layer "F.Cu") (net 8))
 (segment (start 169.612 94.22) (end 172.392 97) (width 0.2) (layer "F.Cu") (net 8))
 (segment (start 143.892 95.39) (end 145.062 94.22) (width 0.2) (layer "F.Cu") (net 8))
 (segment (start 172.392 97) (end 184 97) (width 0.2) (layer "F.Cu") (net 8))
 (segment (start 169.421 89.4964) (end 168.875 88.95) (width 0.2) (layer "F.Cu") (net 34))
 (segment (start 171.276 89.4964) (end 169.421 89.4964) (width 0.2) (layer "F.Cu") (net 34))
 (via (at 171.276 89.4964) (size 0.6) (drill 0.3) (layers "F.Cu" "B.Cu") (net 34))
 (segment (start 171.276 89.4964) (end 171.43 89.3421) (width 0.2) (layer "B.Cu") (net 34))
 (segment (start 171.43 77.6304) (end 170.8 77) (width 0.2) (layer "B.Cu") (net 34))
 (segment (start 171.43 89.3421) (end 171.43 77.6304) (width 0.2) (layer "B.Cu") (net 34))
 (segment (start 181.368 80.5432) (end 174.098 87.8125) (width 0.2) (layer "F.Cu") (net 11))
 (segment (start 181.6325 67.5) (end 181.632 67.5) (width 0.2) (layer "F.Cu") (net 11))
 (segment (start 162.362 65.6) (end 163 65.6) (width 0.2) (layer "F.Cu") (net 11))
 (segment (start 169.385 92.8201) (end 163.87 92.8201) (width 0.2) (layer "F.Cu") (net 11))
 (segment (start 171.387 87) (end 170.829 86.4413) (width 0.2) (layer "F.Cu") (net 11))
 (segment (start 159.132 62.37) (end 162.362 65.6) (width 0.2) (layer "F.Cu") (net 11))
 (segment (start 172.812 87.8125) (end 172 87) (width 0.2) (layer "F.Cu") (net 11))
 (segment (start 181.368 79.5) (end 181.368 80.5432) (width 0.2) (layer "F.Cu") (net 11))
 (segment (start 174.098 87.8125) (end 172.812 87.8125) (width 0.2) (layer "F.Cu") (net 11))
 (segment (start 181.3675 79.5) (end 181.368 79.5) (width 0.2) (layer "F.Cu") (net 11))
 (segment (start 170.656 94.0907) (end 169.385 92.8201) (width 0.2) (layer "F.Cu") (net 11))
 (segment (start 158.03 62.37) (end 159.132 62.37) (width 0.2) (layer "F.Cu") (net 11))
 (segment (start 164.9 67.5) (end 163 65.6) (width 0.2) (layer "F.Cu") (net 11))
 (segment (start 172 87) (end 171.387 87) (width 0.2) (layer "F.Cu") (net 11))
 (segment (start 181.632 67.5) (end 164.9 67.5) (width 0.2) (layer "F.Cu") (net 11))
 (segment (start 163.87 92.8201) (end 162.05 91) (width 0.2) (layer "F.Cu") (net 11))
 (via (at 170.656 94.0907) (size 0.6) (drill 0.3) (layers "F.Cu" "B.Cu") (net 11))
 (via (at 170.829 86.4413) (size 0.6) (drill 0.3) (layers "F.Cu" "B.Cu") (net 11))
 (segment (start 181.632 67.5) (end 182.4495 68.317) (width 0.2) (layer "B.Cu") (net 11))
 (segment (start 183.267 77.6009) (end 181.368 79.5) (width 0.2) (layer "B.Cu") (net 11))
 (segment (start 170.782 90.0966) (end 170.782 93.9652) (width 0.2) (layer "B.Cu") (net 11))
 (segment (start 181.3675 79.5) (end 181.368 79.5) (width 0.2) (layer "B.Cu") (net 11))
 (segment (start 170.782 93.9652) (end 170.656 94.0907) (width 0.2) (layer "B.Cu") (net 11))
 (segment (start 183.267 69.1341) (end 183.267 77.6009) (width 0.2) (layer "B.Cu") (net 11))
 (segment (start 182.4495 68.317) (end 183.267 69.1341) (width 0.2) (layer "B.Cu") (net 11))
 (segment (start 170.829 86.4413) (end 170.631 86.6386) (width 0.2) (layer "B.Cu") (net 11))
 (segment (start 170.631 89.9465) (end 170.782 90.0966) (width 0.2) (layer "B.Cu") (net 11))
 (segment (start 181.6325 67.5) (end 182.4495 68.317) (width 0.2) (layer "B.Cu") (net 11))
 (segment (start 170.631 86.6386) (end 170.631 89.9465) (width 0.2) (layer "B.Cu") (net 11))
 (segment (start 163.089 80.7658) (end 163.089 98.3012) (width 0.2) (layer "B.Cu") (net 5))
 (segment (start 181.4948 62.5) (end 181.355 62.5) (width 0.2) (layer "B.Cu") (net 5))
 (segment (start 181.632 62.5) (end 181.4948 62.5) (width 0.2) (layer "B.Cu") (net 5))
 (segment (start 163.089 98.3012) (end 161.65 99.74) (width 0.2) (layer "B.Cu") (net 5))
 (segment (start 181.355 62.5) (end 163.089 80.7658) (width 0.2) (layer "B.Cu") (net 5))
 (segment (start 181.6325 62.5) (end 181.4948 62.5) (width 0.2) (layer "B.Cu") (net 5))
 (segment (start 166.86 80.21) (end 162.044 80.21) (width 0.2) (layer "F.Cu") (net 4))
 (segment (start 173.65 87) (end 166.86 80.21) (width 0.2) (layer "F.Cu") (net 4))
 (via (at 162.044 80.21) (size 0.6) (drill 0.3) (layers "F.Cu" "B.Cu") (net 4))
 (segment (start 162.044 80.21) (end 161.65 80.6044) (width 0.2) (layer "B.Cu") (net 4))
 (segment (start 161.65 80.6044) (end 161.65 97.2) (width 0.2) (layer "B.Cu") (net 4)))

